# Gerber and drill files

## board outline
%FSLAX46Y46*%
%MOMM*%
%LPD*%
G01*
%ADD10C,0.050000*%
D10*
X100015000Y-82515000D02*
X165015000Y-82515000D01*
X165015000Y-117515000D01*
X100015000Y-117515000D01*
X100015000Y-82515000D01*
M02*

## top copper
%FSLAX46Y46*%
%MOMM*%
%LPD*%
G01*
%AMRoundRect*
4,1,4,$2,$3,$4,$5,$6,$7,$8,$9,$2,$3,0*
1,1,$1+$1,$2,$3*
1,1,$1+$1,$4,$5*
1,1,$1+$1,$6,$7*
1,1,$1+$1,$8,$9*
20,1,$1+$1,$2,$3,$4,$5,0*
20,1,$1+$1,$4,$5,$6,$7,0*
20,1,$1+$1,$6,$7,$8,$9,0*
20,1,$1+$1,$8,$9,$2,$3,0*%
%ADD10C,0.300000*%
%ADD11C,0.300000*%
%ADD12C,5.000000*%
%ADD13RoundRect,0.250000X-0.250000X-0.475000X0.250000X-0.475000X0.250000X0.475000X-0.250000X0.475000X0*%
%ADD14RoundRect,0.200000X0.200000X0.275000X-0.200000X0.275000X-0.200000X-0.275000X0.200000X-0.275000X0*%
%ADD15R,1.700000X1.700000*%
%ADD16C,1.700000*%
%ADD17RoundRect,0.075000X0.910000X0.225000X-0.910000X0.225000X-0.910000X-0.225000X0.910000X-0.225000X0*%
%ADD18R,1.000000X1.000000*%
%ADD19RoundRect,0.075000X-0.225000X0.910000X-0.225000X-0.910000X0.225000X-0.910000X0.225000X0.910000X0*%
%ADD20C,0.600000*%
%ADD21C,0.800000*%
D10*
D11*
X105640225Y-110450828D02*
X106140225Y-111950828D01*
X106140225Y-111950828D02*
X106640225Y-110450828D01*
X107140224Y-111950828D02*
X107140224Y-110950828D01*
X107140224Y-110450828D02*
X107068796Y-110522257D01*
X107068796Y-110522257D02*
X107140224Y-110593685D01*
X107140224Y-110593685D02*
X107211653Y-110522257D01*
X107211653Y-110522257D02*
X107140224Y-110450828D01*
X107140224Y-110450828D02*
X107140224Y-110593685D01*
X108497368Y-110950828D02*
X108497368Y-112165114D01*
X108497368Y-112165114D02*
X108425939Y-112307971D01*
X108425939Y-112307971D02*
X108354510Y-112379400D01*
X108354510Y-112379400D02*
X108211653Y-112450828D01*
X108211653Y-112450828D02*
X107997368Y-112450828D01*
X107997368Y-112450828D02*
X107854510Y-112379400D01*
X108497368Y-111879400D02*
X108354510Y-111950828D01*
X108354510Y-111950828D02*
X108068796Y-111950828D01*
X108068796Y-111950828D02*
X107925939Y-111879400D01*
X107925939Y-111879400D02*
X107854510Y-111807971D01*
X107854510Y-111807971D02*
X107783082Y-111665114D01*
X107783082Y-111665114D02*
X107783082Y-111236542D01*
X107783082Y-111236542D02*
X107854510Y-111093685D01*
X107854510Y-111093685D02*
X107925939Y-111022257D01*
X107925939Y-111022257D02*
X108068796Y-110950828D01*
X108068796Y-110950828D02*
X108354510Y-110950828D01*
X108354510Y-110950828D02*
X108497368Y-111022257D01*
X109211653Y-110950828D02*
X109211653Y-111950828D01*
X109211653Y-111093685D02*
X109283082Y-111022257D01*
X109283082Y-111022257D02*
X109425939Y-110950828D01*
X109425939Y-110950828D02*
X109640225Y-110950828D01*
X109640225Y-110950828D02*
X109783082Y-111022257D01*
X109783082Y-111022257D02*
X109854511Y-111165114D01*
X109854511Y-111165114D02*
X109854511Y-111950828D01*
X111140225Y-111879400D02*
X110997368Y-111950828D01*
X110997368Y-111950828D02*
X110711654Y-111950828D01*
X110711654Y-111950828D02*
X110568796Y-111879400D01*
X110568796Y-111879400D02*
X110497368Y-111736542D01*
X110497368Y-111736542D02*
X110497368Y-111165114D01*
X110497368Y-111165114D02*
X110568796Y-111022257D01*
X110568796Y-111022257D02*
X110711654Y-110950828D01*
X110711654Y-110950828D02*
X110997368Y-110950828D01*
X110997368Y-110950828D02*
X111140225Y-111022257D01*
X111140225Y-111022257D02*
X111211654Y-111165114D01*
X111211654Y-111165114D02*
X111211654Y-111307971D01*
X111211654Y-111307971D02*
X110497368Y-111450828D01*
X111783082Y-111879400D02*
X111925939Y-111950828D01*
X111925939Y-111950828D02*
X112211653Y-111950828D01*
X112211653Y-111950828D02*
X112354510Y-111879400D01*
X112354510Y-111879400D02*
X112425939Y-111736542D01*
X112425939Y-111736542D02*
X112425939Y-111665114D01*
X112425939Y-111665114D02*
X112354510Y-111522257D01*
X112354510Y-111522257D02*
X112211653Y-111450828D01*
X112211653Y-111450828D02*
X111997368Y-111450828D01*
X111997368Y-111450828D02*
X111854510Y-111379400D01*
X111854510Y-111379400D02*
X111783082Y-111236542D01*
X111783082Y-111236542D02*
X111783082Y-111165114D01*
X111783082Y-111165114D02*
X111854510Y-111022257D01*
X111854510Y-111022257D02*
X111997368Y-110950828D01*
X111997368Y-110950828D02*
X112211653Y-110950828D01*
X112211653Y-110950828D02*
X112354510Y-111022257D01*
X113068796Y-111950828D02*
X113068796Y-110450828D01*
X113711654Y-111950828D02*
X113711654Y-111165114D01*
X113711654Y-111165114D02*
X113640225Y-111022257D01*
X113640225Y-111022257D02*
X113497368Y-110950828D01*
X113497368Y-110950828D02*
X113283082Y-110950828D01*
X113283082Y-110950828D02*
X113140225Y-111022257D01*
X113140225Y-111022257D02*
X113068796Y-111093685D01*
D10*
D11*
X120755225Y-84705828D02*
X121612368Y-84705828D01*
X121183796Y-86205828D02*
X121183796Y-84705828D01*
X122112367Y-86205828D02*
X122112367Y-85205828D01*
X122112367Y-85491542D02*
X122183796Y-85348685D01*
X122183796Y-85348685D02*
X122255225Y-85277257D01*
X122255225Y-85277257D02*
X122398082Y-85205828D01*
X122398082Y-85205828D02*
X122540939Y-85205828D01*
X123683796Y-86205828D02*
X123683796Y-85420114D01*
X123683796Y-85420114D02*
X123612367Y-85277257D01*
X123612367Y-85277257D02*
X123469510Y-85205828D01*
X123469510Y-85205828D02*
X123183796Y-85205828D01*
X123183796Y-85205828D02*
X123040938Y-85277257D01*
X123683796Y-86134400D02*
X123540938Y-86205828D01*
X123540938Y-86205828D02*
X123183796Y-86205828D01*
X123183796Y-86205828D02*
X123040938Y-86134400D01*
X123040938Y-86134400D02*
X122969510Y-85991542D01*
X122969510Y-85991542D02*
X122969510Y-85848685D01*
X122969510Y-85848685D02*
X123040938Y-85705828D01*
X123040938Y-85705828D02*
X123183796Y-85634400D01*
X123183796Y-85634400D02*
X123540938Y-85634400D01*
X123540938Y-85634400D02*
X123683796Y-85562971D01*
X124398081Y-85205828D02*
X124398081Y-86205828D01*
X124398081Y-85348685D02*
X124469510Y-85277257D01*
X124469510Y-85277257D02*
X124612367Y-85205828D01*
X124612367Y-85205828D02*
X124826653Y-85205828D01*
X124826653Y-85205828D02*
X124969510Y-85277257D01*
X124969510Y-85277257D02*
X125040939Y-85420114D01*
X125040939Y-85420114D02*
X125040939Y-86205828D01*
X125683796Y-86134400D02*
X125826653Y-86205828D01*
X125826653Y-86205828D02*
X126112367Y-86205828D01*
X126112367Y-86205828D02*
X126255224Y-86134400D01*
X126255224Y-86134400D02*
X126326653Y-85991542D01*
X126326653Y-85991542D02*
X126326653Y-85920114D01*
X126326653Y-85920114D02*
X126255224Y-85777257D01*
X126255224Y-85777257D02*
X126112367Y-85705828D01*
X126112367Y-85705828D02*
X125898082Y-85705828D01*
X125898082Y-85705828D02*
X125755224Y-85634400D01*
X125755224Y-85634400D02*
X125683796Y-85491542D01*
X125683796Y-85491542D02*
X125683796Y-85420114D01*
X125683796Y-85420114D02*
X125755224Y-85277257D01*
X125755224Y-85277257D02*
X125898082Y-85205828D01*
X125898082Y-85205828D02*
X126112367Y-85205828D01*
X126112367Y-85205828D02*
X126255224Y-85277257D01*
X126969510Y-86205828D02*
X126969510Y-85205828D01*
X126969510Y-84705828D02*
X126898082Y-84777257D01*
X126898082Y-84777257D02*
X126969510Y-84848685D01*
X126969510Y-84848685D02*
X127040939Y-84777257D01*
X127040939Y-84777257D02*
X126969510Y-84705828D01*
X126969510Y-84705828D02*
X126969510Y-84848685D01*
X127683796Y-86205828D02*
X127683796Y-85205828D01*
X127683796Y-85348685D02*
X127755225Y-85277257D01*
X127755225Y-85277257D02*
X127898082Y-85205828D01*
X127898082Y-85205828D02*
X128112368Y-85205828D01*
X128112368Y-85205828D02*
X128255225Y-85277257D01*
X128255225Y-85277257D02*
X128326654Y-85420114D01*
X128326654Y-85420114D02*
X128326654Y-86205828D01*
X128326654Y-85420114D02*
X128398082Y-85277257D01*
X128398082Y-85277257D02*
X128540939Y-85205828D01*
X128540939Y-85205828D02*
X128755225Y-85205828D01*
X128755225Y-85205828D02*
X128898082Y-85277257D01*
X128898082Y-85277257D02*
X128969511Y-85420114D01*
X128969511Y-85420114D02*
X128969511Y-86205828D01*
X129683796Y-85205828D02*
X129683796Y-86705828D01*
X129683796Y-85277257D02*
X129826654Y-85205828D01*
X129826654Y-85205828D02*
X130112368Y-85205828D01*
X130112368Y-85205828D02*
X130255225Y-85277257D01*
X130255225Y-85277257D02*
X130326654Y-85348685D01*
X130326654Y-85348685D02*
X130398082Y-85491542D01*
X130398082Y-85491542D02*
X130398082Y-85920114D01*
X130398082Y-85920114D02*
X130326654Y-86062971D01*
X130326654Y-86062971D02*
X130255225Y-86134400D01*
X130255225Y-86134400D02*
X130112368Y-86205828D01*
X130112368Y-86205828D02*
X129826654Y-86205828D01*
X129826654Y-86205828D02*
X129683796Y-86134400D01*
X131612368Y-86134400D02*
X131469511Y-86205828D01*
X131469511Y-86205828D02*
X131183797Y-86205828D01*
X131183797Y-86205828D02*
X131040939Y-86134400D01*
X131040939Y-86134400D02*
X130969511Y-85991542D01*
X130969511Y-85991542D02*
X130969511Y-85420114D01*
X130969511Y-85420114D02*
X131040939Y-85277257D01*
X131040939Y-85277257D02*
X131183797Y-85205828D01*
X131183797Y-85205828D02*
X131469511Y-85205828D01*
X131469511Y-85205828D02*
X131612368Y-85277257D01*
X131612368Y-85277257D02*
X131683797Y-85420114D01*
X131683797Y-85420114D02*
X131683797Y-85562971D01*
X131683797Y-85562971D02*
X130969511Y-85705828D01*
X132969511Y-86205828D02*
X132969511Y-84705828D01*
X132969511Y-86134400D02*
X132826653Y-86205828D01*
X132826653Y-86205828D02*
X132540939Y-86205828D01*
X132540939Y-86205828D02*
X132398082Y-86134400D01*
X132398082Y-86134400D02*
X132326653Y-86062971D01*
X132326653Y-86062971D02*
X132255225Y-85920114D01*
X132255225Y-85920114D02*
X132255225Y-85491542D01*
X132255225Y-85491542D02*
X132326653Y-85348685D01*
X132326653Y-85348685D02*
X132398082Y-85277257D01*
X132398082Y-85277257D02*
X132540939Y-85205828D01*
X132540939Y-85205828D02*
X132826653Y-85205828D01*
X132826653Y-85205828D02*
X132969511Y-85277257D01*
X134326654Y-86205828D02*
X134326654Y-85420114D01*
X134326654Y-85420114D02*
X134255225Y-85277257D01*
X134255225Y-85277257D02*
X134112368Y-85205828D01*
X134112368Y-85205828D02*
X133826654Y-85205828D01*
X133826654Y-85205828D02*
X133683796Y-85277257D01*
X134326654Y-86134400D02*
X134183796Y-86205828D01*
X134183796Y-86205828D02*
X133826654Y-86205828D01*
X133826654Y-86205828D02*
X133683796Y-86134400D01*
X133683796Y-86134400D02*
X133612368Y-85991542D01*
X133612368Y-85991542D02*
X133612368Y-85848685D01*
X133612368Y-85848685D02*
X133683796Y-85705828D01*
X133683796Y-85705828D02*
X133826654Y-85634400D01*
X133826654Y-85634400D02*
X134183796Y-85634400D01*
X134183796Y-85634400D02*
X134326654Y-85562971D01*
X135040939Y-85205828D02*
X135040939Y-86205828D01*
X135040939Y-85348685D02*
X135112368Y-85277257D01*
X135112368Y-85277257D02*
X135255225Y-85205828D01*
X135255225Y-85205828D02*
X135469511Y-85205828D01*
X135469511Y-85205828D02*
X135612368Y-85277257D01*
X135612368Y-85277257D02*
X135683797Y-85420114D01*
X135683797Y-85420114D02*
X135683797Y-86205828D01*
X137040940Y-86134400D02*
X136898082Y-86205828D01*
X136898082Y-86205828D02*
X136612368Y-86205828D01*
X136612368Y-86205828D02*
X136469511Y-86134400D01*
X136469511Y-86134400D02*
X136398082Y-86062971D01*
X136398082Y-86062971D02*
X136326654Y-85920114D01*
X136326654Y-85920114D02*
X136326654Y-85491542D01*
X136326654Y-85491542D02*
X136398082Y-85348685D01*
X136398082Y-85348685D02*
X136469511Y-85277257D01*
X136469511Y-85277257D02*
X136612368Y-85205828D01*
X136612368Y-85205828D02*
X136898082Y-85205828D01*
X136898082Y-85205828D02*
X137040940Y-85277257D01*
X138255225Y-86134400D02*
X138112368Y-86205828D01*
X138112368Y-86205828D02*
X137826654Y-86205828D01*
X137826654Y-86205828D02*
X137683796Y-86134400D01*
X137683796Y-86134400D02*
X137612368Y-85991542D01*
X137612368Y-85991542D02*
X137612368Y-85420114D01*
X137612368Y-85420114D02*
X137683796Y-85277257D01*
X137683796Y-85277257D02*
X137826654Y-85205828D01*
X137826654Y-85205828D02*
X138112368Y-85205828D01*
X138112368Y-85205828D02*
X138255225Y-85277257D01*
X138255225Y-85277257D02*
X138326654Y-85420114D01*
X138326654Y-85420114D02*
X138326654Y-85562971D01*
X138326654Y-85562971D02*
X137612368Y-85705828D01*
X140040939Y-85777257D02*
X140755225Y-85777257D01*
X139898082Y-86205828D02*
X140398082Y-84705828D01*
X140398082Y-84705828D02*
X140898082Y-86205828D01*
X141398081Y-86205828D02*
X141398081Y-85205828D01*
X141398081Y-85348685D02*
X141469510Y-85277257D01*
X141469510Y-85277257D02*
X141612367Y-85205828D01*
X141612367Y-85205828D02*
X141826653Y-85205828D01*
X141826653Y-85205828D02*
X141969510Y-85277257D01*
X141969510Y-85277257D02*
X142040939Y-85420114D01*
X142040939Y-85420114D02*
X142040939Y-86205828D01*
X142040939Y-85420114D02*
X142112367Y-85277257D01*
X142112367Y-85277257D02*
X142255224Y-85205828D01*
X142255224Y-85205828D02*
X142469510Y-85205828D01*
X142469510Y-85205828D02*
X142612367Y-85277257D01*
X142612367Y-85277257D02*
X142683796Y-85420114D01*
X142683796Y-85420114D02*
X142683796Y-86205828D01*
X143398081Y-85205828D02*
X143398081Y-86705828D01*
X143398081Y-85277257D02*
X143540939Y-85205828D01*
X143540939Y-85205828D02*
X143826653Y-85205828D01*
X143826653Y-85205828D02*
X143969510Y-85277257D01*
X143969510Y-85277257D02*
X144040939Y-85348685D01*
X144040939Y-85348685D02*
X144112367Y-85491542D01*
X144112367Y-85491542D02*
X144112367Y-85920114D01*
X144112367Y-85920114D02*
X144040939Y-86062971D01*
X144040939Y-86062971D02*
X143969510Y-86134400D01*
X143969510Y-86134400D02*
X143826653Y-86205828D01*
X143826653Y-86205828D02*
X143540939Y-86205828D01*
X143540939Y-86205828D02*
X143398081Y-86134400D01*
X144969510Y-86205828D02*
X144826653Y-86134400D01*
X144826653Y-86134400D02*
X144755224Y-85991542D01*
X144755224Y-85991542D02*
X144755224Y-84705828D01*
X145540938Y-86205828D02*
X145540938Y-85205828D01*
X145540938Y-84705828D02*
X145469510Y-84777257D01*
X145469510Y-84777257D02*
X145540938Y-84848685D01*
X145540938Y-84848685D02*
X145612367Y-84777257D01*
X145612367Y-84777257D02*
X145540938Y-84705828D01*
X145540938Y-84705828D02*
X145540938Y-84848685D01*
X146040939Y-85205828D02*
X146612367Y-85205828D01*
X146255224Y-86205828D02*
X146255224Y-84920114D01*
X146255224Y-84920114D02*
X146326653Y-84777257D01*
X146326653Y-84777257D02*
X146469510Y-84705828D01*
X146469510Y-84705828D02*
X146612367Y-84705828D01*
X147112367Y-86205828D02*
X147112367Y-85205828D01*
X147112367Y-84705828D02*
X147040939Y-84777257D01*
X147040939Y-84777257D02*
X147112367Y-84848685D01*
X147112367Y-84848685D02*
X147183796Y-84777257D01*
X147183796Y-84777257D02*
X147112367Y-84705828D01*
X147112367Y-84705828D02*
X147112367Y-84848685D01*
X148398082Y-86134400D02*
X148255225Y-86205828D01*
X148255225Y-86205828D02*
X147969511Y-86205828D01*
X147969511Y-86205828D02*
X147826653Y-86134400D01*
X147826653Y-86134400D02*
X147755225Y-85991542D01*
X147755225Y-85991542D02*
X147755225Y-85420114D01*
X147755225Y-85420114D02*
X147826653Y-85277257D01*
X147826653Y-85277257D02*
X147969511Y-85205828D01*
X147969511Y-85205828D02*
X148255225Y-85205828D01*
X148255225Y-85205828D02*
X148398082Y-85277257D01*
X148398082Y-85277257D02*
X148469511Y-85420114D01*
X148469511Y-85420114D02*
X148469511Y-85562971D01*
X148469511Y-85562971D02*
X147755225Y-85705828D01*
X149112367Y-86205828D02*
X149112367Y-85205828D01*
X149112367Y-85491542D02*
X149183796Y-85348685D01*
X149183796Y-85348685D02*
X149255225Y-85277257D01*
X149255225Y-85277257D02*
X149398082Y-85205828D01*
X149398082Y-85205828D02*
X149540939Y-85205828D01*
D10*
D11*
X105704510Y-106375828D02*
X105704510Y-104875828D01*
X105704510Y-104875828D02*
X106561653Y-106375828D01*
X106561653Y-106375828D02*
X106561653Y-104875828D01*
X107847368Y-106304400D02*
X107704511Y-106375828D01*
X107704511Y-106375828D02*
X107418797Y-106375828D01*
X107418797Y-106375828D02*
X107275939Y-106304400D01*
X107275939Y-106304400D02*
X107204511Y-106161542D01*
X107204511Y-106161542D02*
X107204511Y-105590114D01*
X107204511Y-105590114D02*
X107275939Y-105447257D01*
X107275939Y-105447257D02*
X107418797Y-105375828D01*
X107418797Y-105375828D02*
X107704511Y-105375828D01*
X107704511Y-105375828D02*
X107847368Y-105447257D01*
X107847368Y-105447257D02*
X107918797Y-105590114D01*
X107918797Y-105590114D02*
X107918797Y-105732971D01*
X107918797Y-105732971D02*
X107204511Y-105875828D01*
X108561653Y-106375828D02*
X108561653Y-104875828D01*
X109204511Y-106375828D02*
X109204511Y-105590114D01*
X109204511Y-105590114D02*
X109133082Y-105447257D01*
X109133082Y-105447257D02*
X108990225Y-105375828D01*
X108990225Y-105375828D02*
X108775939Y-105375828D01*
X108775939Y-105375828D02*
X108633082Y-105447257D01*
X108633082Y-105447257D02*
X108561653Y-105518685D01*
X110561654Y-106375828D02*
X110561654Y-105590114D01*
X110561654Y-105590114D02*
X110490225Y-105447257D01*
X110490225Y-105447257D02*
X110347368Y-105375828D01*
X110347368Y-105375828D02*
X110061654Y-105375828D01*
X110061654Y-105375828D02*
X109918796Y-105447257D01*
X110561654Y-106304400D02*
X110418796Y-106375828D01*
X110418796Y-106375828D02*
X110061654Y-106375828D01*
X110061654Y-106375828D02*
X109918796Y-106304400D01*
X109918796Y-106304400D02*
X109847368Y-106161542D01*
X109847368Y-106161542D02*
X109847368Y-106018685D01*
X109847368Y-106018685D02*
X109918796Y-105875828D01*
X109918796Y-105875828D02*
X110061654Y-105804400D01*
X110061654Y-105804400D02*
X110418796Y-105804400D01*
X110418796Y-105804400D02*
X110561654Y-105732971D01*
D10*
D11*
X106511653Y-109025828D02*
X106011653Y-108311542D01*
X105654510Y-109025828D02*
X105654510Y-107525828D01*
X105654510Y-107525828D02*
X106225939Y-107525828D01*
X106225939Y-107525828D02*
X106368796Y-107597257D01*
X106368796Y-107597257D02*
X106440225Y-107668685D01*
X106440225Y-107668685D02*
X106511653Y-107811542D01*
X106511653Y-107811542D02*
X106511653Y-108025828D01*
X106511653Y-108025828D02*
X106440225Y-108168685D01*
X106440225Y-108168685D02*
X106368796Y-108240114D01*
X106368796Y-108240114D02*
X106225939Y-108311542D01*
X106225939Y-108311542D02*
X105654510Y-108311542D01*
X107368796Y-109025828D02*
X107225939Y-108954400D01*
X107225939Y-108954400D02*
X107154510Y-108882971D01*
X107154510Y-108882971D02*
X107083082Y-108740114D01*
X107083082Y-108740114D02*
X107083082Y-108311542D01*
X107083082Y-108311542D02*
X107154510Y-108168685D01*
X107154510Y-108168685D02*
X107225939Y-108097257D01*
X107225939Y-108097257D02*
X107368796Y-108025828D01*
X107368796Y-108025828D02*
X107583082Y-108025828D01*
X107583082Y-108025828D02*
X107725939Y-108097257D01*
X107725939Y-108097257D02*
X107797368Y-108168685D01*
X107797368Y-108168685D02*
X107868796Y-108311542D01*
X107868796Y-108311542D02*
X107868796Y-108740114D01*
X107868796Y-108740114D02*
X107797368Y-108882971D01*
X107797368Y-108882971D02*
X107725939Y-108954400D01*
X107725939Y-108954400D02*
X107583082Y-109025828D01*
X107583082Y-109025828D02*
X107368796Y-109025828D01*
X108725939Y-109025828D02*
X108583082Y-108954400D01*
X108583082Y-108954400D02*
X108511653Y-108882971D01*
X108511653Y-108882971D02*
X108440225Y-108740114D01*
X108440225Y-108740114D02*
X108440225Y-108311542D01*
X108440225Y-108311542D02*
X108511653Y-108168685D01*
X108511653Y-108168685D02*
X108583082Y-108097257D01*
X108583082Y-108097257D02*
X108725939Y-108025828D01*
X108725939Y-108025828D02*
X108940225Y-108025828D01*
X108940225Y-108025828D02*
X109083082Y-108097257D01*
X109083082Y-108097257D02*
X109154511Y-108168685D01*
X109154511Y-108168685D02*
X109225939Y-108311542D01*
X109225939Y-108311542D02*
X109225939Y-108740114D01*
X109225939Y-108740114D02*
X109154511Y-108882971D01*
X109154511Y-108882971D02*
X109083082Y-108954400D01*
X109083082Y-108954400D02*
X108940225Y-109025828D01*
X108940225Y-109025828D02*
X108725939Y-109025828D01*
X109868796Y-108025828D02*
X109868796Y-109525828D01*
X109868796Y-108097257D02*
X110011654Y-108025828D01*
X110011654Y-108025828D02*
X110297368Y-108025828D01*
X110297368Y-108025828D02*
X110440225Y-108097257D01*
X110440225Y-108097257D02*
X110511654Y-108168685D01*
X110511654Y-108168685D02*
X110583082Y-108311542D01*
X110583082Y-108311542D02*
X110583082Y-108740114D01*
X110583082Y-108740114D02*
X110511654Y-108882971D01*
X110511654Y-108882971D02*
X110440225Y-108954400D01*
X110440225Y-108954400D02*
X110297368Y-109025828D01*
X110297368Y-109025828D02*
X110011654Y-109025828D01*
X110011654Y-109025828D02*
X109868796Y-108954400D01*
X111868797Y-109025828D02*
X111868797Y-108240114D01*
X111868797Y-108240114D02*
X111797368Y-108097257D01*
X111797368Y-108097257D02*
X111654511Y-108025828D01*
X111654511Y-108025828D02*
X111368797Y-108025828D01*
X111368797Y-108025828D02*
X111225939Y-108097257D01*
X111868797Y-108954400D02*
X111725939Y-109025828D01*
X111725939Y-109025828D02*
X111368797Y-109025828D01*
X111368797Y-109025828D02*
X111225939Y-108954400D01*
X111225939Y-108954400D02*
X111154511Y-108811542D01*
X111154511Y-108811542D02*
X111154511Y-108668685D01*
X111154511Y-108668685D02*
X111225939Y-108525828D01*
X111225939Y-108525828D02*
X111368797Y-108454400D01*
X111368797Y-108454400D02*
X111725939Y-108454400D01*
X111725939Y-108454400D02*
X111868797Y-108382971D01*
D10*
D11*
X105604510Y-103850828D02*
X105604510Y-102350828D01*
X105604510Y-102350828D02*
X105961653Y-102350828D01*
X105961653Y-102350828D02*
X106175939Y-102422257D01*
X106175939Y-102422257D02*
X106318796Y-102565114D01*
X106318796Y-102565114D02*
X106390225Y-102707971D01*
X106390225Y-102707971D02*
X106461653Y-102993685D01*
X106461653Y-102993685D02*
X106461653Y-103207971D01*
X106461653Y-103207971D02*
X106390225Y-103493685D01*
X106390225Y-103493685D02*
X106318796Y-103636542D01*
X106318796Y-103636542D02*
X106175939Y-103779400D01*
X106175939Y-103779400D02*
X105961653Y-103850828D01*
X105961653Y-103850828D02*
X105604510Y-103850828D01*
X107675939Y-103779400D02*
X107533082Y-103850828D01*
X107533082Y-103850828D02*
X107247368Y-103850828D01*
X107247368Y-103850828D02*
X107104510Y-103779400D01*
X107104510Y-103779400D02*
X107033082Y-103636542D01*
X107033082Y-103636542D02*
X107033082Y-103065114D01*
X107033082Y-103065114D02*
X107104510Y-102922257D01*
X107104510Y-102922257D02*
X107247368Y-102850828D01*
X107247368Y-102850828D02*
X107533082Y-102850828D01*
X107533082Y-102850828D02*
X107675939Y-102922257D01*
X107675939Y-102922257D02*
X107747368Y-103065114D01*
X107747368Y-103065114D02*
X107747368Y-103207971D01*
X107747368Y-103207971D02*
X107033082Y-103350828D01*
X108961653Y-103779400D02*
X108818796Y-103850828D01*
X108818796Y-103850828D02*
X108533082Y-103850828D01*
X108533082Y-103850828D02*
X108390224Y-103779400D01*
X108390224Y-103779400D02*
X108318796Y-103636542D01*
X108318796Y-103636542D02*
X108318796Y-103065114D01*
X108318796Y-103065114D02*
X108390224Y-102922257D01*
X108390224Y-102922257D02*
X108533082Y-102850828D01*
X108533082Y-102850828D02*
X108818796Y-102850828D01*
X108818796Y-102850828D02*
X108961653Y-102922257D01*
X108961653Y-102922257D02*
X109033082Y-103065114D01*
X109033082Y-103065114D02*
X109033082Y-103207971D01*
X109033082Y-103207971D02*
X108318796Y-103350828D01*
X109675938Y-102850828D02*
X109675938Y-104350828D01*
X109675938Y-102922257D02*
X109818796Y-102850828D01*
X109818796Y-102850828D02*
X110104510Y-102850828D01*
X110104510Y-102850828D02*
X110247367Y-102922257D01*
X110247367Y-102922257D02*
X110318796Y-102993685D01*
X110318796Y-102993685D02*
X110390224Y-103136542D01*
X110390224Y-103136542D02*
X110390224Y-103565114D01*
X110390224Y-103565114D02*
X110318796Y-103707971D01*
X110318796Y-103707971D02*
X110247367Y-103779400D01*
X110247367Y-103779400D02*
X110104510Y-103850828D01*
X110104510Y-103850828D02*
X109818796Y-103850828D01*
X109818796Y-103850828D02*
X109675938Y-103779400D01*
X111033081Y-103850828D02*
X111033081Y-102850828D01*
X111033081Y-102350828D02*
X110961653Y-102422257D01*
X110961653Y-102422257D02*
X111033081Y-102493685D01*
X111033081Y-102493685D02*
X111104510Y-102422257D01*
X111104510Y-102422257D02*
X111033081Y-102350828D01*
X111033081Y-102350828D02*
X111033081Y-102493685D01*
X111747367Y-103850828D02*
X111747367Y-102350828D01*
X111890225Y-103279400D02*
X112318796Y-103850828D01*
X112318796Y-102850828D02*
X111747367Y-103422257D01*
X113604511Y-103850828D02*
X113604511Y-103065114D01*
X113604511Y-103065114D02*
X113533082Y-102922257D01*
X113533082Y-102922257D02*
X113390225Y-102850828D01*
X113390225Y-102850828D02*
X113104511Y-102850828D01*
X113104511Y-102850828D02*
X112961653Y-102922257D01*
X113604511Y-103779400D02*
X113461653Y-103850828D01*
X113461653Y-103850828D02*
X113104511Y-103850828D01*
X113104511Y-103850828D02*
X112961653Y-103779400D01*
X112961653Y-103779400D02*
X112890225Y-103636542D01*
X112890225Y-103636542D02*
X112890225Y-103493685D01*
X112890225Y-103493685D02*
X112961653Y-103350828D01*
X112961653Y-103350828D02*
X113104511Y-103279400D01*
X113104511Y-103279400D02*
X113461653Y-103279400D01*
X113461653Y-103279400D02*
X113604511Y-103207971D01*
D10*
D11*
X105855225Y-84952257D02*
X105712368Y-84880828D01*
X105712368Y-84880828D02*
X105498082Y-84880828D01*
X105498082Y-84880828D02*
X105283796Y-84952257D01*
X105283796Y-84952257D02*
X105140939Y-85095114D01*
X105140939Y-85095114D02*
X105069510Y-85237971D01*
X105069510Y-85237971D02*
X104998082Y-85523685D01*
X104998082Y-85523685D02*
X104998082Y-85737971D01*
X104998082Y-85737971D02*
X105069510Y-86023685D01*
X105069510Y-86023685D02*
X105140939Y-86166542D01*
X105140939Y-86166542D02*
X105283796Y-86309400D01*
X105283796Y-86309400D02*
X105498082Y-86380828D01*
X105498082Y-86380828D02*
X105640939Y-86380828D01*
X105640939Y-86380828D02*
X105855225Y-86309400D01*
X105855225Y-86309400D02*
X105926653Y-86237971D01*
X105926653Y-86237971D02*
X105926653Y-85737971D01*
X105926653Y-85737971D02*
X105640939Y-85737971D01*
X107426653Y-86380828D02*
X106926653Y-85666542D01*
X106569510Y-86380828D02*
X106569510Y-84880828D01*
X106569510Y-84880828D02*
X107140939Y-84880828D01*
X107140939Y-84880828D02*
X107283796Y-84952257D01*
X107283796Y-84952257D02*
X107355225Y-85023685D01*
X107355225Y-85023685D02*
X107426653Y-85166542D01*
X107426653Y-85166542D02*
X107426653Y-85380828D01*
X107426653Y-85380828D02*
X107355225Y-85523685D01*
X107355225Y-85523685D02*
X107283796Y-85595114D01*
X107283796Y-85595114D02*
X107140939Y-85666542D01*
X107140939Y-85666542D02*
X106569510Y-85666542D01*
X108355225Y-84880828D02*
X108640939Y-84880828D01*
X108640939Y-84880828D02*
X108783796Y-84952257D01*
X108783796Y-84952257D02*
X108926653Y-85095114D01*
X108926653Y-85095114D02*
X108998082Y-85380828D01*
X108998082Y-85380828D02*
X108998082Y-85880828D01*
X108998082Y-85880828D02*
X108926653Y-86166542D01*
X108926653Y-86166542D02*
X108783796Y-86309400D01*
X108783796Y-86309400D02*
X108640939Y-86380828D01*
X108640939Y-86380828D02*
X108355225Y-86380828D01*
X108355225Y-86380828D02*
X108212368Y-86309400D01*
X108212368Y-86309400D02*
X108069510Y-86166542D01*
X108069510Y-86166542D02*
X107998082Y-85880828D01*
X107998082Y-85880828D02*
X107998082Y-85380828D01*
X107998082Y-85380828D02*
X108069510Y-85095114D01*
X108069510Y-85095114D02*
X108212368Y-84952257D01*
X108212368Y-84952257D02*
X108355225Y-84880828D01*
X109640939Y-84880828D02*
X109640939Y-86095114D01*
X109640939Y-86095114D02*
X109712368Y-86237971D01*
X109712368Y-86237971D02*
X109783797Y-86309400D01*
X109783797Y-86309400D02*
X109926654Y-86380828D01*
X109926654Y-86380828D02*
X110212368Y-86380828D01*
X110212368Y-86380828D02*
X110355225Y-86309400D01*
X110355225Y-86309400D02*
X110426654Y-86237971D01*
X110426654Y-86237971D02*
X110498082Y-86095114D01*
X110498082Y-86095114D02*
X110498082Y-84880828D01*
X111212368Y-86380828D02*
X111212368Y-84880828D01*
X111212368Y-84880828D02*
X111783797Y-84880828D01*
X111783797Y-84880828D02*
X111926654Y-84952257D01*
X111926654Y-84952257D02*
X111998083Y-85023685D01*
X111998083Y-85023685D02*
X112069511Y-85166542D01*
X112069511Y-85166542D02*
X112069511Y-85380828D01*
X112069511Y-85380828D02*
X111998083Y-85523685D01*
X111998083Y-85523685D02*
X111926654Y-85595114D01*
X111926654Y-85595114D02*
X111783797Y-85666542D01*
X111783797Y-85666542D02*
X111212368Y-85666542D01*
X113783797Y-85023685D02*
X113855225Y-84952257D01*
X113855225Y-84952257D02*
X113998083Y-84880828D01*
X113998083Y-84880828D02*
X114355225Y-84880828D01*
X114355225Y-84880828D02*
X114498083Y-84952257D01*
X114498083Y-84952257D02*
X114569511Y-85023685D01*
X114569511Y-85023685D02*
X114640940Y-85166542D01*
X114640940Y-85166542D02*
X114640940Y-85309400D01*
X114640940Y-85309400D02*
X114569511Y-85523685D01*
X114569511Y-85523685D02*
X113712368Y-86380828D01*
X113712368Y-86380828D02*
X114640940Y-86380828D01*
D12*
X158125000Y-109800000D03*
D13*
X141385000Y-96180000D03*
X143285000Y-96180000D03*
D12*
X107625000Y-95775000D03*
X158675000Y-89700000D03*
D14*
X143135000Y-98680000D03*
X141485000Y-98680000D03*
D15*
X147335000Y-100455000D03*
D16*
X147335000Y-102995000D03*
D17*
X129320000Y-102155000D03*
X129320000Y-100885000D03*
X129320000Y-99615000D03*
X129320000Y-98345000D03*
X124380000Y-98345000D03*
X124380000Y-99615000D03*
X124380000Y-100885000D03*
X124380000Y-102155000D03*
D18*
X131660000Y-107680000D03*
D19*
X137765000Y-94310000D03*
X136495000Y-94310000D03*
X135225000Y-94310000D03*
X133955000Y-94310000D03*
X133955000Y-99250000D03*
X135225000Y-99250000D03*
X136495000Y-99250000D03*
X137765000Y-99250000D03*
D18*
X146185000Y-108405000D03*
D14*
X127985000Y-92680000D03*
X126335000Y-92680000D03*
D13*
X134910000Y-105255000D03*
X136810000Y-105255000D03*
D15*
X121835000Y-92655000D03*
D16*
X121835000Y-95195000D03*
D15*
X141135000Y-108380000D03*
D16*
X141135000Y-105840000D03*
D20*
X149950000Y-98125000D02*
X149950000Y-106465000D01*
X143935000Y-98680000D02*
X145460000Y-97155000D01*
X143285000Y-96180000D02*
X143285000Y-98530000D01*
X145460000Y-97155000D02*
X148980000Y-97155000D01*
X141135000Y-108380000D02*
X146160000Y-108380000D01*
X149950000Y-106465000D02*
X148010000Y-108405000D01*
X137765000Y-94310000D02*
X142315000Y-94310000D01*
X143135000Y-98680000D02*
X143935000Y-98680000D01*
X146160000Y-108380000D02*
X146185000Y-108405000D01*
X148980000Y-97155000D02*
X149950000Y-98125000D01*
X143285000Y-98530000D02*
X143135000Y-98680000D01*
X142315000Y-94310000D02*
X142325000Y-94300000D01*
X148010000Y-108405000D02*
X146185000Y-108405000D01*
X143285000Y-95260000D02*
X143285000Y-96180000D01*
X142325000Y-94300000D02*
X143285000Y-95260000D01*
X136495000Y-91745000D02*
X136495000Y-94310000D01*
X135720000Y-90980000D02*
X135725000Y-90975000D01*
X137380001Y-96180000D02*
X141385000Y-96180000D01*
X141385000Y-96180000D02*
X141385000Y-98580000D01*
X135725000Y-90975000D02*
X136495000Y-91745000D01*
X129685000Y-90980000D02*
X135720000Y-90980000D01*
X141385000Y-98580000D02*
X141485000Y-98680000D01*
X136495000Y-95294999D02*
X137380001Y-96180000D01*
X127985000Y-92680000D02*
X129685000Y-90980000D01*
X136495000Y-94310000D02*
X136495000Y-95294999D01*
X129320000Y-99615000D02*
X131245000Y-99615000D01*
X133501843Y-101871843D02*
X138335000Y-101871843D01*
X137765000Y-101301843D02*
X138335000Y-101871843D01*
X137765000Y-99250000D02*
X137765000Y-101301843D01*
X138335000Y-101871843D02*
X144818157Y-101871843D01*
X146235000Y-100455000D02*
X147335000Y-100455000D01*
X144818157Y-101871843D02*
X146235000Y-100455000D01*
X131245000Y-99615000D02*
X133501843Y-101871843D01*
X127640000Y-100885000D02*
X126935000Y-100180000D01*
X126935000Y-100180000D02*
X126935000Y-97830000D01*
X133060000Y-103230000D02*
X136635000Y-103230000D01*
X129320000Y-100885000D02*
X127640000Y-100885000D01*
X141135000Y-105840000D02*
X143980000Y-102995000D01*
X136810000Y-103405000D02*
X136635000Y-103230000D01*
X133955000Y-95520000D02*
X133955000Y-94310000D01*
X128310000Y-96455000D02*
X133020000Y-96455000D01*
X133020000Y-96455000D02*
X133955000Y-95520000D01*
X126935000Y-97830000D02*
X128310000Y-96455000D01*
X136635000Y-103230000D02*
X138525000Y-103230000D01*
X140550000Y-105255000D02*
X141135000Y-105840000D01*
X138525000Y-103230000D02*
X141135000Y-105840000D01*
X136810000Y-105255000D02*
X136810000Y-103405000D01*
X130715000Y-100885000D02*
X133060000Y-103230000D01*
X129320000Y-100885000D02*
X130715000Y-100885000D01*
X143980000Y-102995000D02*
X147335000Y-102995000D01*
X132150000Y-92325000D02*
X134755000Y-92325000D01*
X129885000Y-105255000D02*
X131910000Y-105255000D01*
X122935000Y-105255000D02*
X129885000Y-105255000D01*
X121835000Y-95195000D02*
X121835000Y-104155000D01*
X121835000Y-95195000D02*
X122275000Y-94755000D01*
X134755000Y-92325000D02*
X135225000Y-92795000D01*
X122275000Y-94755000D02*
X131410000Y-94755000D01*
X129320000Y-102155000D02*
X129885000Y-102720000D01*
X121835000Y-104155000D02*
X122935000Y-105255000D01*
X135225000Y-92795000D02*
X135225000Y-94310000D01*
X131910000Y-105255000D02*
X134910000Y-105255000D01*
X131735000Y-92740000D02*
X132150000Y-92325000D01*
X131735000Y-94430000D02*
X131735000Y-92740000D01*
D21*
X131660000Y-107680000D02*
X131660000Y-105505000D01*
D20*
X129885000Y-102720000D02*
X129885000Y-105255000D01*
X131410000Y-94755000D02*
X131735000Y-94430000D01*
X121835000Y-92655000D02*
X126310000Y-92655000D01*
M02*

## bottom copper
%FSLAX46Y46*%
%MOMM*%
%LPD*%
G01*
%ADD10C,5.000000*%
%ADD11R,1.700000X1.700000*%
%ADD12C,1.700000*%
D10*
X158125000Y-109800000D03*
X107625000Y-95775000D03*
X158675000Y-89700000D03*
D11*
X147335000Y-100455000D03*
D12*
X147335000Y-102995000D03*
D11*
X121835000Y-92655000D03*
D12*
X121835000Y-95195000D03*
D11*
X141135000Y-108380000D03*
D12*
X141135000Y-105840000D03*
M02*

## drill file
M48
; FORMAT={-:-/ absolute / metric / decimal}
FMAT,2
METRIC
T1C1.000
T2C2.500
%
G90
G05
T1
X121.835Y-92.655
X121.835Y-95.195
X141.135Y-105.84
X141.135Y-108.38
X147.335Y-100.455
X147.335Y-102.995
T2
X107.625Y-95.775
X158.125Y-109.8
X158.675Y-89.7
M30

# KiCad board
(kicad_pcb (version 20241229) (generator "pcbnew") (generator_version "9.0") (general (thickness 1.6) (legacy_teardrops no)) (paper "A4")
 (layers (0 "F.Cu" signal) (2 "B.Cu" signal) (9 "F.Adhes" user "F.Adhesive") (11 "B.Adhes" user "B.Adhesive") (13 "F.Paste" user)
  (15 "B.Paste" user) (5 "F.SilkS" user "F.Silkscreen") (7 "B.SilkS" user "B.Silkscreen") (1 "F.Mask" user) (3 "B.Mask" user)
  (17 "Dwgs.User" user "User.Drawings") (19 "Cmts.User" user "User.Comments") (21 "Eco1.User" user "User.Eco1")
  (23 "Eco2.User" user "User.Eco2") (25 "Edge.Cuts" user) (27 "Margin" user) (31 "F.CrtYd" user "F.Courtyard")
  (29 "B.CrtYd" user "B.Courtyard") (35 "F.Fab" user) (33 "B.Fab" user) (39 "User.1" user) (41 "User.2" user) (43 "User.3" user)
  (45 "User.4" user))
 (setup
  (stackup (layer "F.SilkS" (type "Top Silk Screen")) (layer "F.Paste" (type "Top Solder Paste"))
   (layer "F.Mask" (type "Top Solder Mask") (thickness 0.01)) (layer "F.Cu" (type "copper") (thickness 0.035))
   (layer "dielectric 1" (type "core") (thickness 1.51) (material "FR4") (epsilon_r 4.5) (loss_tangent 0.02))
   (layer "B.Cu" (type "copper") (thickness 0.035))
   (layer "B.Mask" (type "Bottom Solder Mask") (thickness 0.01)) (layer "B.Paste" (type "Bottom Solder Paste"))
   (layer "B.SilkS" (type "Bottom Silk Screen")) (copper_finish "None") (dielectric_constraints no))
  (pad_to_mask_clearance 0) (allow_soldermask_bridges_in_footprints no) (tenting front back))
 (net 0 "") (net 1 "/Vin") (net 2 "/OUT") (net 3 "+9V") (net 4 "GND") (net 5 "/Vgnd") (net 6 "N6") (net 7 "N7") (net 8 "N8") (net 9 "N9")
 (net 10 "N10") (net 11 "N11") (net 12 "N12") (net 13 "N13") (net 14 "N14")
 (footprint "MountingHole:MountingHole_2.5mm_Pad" (layer "F.Cu") (at 158.125 109.8)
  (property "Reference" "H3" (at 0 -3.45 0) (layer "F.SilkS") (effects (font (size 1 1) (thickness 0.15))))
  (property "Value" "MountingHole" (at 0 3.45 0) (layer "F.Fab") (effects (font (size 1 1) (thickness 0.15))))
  (pad "1" thru_hole circle (at 0 0) (size 5 5) (drill 2.5) (layers "*.Cu" "*.Mask") (remove_unused_layers no) (zone_connect 2)))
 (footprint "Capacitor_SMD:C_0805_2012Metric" (layer "F.Cu") (at 142.335 96.18)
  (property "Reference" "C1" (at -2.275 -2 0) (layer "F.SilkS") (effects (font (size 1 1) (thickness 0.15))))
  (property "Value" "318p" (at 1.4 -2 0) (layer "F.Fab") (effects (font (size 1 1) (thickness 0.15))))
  (pad "1" smd roundrect (at -0.95 0) (size 1 1.45) (layers "F.Cu" "F.Mask" "F.Paste") (roundrect_rratio 0.25) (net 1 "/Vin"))
  (pad "2" smd roundrect (at 0.95 0) (size 1 1.45) (layers "F.Cu" "F.Mask" "F.Paste") (roundrect_rratio 0.25) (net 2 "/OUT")))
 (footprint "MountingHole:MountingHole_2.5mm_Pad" (layer "F.Cu") (at 107.625 95.775)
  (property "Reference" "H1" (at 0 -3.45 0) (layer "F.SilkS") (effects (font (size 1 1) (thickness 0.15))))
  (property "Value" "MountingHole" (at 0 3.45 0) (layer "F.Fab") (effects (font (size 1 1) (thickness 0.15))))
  (pad "1" thru_hole circle (at 0 0) (size 5 5) (drill 2.5) (layers "*.Cu" "*.Mask") (remove_unused_layers no) (zone_connect 2)))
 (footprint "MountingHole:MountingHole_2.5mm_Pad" (layer "F.Cu") (at 158.675 89.7)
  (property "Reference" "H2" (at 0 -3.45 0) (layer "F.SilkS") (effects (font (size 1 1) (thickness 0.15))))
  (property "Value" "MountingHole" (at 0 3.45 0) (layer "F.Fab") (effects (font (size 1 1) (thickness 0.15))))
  (pad "1" thru_hole circle (at 0 0) (size 5 5) (drill 2.5) (layers "*.Cu" "*.Mask") (remove_unused_layers no) (zone_connect 2)))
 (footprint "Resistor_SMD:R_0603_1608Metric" (layer "F.Cu") (at 142.31 98.68 180)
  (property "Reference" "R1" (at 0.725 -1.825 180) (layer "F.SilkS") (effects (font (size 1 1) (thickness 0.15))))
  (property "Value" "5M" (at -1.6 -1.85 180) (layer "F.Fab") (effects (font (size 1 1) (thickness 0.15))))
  (pad "1" smd roundrect (at -0.825 0 180) (size 0.8 0.95) (layers "F.Cu" "F.Mask" "F.Paste") (roundrect_rratio 0.25) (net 2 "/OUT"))
  (pad "2" smd roundrect (at 0.825 0 180) (size 0.8 0.95) (layers "F.Cu" "F.Mask" "F.Paste") (roundrect_rratio 0.25) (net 1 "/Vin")))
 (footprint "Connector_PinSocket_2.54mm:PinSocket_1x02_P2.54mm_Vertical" (layer "F.Cu") (at 147.335 100.455)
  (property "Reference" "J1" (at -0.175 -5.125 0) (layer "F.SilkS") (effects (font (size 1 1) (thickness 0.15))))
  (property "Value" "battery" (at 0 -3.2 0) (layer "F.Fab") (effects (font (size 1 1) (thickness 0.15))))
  (pad "1" thru_hole rect (at 0 0) (size 1.7 1.7) (drill 1) (layers "*.Cu" "*.Mask") (remove_unused_layers no) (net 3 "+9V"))
  (pad "2" thru_hole circle (at 0 2.54) (size 1.7 1.7) (drill 1) (layers "*.Cu" "*.Mask") (remove_unused_layers no) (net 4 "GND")))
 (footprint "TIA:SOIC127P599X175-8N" (layer "F.Cu") (at 126.85 100.25 180)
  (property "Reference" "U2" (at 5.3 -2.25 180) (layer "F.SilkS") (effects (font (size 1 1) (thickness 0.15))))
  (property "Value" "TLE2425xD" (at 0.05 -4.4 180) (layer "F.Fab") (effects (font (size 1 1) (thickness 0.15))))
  (pad "1" smd roundrect (at -2.47 -1.905 180) (size 1.97 0.6) (layers "F.Cu" "F.Mask" "F.Paste") (roundrect_rratio 0.125) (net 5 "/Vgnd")
   (solder_mask_margin 0.102))
  (pad "2" smd roundrect (at -2.47 -0.635 180) (size 1.97 0.6) (layers "F.Cu" "F.Mask" "F.Paste") (roundrect_rratio 0.125) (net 4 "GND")
   (solder_mask_margin 0.102))
  (pad "3" smd roundrect (at -2.47 0.635 180) (size 1.97 0.6) (layers "F.Cu" "F.Mask" "F.Paste") (roundrect_rratio 0.125) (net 3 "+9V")
   (solder_mask_margin 0.102))
  (pad "4" smd roundrect (at -2.47 1.905 180) (size 1.97 0.6) (layers "F.Cu" "F.Mask" "F.Paste") (roundrect_rratio 0.125) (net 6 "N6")
   (solder_mask_margin 0.102))
  (pad "5" smd roundrect (at 2.47 1.905 180) (size 1.97 0.6) (layers "F.Cu" "F.Mask" "F.Paste") (roundrect_rratio 0.125) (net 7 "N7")
   (solder_mask_margin 0.102))
  (pad "6" smd roundrect (at 2.47 0.635 180) (size 1.97 0.6) (layers "F.Cu" "F.Mask" "F.Paste") (roundrect_rratio 0.125) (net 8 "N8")
   (solder_mask_margin 0.102))
  (pad "7" smd roundrect (at 2.47 -0.635 180) (size 1.97 0.6) (layers "F.Cu" "F.Mask" "F.Paste") (roundrect_rratio 0.125) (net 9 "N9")
   (solder_mask_margin 0.102))
  (pad "8" smd roundrect (at 2.47 -1.905 180) (size 1.97 0.6) (layers "F.Cu" "F.Mask" "F.Paste") (roundrect_rratio 0.125) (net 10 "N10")
   (solder_mask_margin 0.102)))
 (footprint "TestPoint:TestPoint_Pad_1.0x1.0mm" (layer "F.Cu") (at 131.66 107.68 180)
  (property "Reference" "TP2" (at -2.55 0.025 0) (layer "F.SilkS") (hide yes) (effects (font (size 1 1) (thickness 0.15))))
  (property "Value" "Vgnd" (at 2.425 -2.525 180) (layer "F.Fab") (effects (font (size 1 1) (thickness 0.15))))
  (pad "1" smd rect (at 0 0 180) (size 1 1) (layers "F.Cu" "F.Mask") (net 5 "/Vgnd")))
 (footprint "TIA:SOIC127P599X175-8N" (layer "F.Cu") (at 135.86 96.78 -90)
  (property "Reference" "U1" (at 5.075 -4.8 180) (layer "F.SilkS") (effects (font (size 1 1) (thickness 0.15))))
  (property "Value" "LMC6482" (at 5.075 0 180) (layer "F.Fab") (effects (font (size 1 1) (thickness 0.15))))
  (pad "1" smd roundrect (at -2.47 -1.905 270) (size 1.97 0.6) (layers "F.Cu" "F.Mask" "F.Paste") (roundrect_rratio 0.125) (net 2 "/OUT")
   (solder_mask_margin 0.102))
  (pad "2" smd roundrect (at -2.47 -0.635 270) (size 1.97 0.6) (layers "F.Cu" "F.Mask" "F.Paste") (roundrect_rratio 0.125) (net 1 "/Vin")
   (solder_mask_margin 0.102))
  (pad "3" smd roundrect (at -2.47 0.635 270) (size 1.97 0.6) (layers "F.Cu" "F.Mask" "F.Paste") (roundrect_rratio 0.125) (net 5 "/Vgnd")
   (solder_mask_margin 0.102))
  (pad "4" smd roundrect (at -2.47 1.905 270) (size 1.97 0.6) (layers "F.Cu" "F.Mask" "F.Paste") (roundrect_rratio 0.125) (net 4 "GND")
   (solder_mask_margin 0.102))
  (pad "5" smd roundrect (at 2.47 1.905 270) (size 1.97 0.6) (layers "F.Cu" "F.Mask" "F.Paste") (roundrect_rratio 0.125) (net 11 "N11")
   (solder_mask_margin 0.102))
  (pad "6" smd roundrect (at 2.47 0.635 270) (size 1.97 0.6) (layers "F.Cu" "F.Mask" "F.Paste") (roundrect_rratio 0.125) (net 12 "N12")
   (solder_mask_margin 0.102))
  (pad "7" smd roundrect (at 2.47 -0.635 270) (size 1.97 0.6) (layers "F.Cu" "F.Mask" "F.Paste") (roundrect_rratio 0.125) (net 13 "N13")
   (solder_mask_margin 0.102))
  (pad "8" smd roundrect (at 2.47 -1.905 270) (size 1.97 0.6) (layers "F.Cu" "F.Mask" "F.Paste") (roundrect_rratio 0.125) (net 3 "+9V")
   (solder_mask_margin 0.102)))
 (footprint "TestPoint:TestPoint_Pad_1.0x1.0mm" (layer "F.Cu") (at 146.185 108.405)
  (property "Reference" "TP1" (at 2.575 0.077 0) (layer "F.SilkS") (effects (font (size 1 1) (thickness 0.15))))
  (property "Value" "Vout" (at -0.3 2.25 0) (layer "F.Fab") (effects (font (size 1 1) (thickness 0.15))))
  (pad "1" smd rect (at 0 0) (size 1 1) (layers "F.Cu" "F.Mask") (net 2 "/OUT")))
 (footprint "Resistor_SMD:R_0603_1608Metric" (layer "F.Cu") (at 127.16 92.68 180)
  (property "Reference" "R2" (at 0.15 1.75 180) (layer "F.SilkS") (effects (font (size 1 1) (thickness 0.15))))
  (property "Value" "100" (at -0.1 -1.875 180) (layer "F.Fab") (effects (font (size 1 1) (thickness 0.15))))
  (pad "1" smd roundrect (at -0.825 0 180) (size 0.8 0.95) (layers "F.Cu" "F.Mask" "F.Paste") (roundrect_rratio 0.25) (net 1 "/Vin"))
  (pad "2" smd roundrect (at 0.825 0 180) (size 0.8 0.95) (layers "F.Cu" "F.Mask" "F.Paste") (roundrect_rratio 0.25) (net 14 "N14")))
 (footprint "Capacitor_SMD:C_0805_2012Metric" (layer "F.Cu") (at 135.86 105.255)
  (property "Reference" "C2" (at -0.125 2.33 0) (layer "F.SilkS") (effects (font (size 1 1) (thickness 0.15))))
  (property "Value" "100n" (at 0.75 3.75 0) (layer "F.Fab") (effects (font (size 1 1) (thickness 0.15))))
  (pad "1" smd roundrect (at -0.95 0) (size 1 1.45) (layers "F.Cu" "F.Mask" "F.Paste") (roundrect_rratio 0.25) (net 5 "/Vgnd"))
  (pad "2" smd roundrect (at 0.95 0) (size 1 1.45) (layers "F.Cu" "F.Mask" "F.Paste") (roundrect_rratio 0.25) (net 4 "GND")))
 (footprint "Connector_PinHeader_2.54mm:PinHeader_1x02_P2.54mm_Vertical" (layer "F.Cu") (at 121.835 92.655)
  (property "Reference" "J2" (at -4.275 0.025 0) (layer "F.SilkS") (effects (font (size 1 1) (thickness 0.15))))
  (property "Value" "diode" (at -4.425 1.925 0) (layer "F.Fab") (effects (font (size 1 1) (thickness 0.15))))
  (pad "1" thru_hole rect (at 0 0) (size 1.7 1.7) (drill 1) (layers "*.Cu" "*.Mask") (remove_unused_layers no) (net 14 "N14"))
  (pad "2" thru_hole circle (at 0 2.54) (size 1.7 1.7) (drill 1) (layers "*.Cu" "*.Mask") (remove_unused_layers no) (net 5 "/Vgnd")))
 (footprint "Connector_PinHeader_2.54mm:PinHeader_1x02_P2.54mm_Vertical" (layer "F.Cu") (at 141.135 108.38 180)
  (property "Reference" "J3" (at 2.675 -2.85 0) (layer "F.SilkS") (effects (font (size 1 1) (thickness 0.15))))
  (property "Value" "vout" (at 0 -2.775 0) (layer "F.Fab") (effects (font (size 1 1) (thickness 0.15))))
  (pad "1" thru_hole rect (at 0 0 180) (size 1.7 1.7) (drill 1) (layers "*.Cu" "*.Mask") (remove_unused_layers no) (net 2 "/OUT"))
  (pad "2" thru_hole circle (at 0 2.54 180) (size 1.7 1.7) (drill 1) (layers "*.Cu" "*.Mask") (remove_unused_layers no) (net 4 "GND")))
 (gr_rect (start 100.015 82.515) (end 165.015 117.515) (stroke (width 0.05) (type solid)) (fill no) (layer "Edge.Cuts"))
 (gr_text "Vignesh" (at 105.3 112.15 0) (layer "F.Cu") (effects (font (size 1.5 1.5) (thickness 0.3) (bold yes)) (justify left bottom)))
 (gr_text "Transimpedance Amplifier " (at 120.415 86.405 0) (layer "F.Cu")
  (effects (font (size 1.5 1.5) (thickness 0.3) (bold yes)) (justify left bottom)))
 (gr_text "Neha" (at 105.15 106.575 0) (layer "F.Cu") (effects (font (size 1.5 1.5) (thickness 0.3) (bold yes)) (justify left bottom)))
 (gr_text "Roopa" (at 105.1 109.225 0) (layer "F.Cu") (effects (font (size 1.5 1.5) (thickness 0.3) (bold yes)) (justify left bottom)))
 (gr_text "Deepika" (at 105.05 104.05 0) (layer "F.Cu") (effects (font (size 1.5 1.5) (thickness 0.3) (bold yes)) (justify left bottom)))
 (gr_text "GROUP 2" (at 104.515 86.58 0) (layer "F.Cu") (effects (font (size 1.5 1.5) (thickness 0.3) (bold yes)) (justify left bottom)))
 (segment (start 149.95 98.125) (end 149.95 106.465) (width 0.6) (layer "F.Cu") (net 2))
 (segment (start 143.935 98.68) (end 145.46 97.155) (width 0.6) (layer "F.Cu") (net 2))
 (segment (start 143.285 96.18) (end 143.285 98.53) (width 0.6) (layer "F.Cu") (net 2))
 (segment (start 145.46 97.155) (end 148.98 97.155) (width 0.6) (layer "F.Cu") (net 2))
 (segment (start 141.135 108.38) (end 146.16 108.38) (width 0.6) (layer "F.Cu") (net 2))
 (segment (start 149.95 106.465) (end 148.01 108.405) (width 0.6) (layer "F.Cu") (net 2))
 (segment (start 137.765 94.31) (end 142.315 94.31) (width 0.6) (layer "F.Cu") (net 2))
 (segment (start 143.135 98.68) (end 143.935 98.68) (width 0.6) (layer "F.Cu") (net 2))
 (segment (start 146.16 108.38) (end 146.185 108.405) (width 0.6) (layer "F.Cu") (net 2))
 (segment (start 148.98 97.155) (end 149.95 98.125) (width 0.6) (layer "F.Cu") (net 2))
 (segment (start 143.285 98.53) (end 143.135 98.68) (width 0.6) (layer "F.Cu") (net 2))
 (segment (start 142.315 94.31) (end 142.325 94.3) (width 0.6) (layer "F.Cu") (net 2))
 (segment (start 148.01 108.405) (end 146.185 108.405) (width 0.6) (layer "F.Cu") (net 2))
 (segment (start 143.285 95.26) (end 143.285 96.18) (width 0.6) (layer "F.Cu") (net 2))
 (segment (start 142.325 94.3) (end 143.285 95.26) (width 0.6) (layer "F.Cu") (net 2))
 (segment (start 136.495 91.745) (end 136.495 94.31) (width 0.6) (layer "F.Cu") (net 1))
 (segment (start 135.72 90.98) (end 135.725 90.975) (width 0.6) (layer "F.Cu") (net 1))
 (segment (start 137.380001 96.18) (end 141.385 96.18) (width 0.6) (layer "F.Cu") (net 1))
 (segment (start 141.385 96.18) (end 141.385 98.58) (width 0.6) (layer "F.Cu") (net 1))
 (segment (start 135.725 90.975) (end 136.495 91.745) (width 0.6) (layer "F.Cu") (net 1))
 (segment (start 129.685 90.98) (end 135.72 90.98) (width 0.6) (layer "F.Cu") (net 1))
 (segment (start 141.385 98.58) (end 141.485 98.68) (width 0.6) (layer "F.Cu") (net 1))
 (segment (start 136.495 95.294999) (end 137.380001 96.18) (width 0.6) (layer "F.Cu") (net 1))
 (segment (start 127.985 92.68) (end 129.685 90.98) (width 0.6) (layer "F.Cu") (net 1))
 (segment (start 136.495 94.31) (end 136.495 95.294999) (width 0.6) (layer "F.Cu") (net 1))
 (segment (start 129.32 99.615) (end 131.245 99.615) (width 0.6) (layer "F.Cu") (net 3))
 (segment (start 133.501843 101.871843) (end 138.335 101.871843) (width 0.6) (layer "F.Cu") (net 3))
 (segment (start 137.765 101.301843) (end 138.335 101.871843) (width 0.6) (layer "F.Cu") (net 3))
 (segment (start 137.765 99.25) (end 137.765 101.301843) (width 0.6) (layer "F.Cu") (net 3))
 (segment (start 138.335 101.871843) (end 144.818157 101.871843) (width 0.6) (layer "F.Cu") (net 3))
 (segment (start 146.235 100.455) (end 147.335 100.455) (width 0.6) (layer "F.Cu") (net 3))
 (segment (start 144.818157 101.871843) (end 146.235 100.455) (width 0.6) (layer "F.Cu") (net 3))
 (segment (start 131.245 99.615) (end 133.501843 101.871843) (width 0.6) (layer "F.Cu") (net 3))
 (segment (start 127.64 100.885) (end 126.935 100.18) (width 0.6) (layer "F.Cu") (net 4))
 (segment (start 126.935 100.18) (end 126.935 97.83) (width 0.6) (layer "F.Cu") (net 4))
 (segment (start 133.06 103.23) (end 136.635 103.23) (width 0.6) (layer "F.Cu") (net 4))
 (segment (start 129.32 100.885) (end 127.64 100.885) (width 0.6) (layer "F.Cu") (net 4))
 (segment (start 141.135 105.84) (end 143.98 102.995) (width 0.6) (layer "F.Cu") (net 4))
 (segment (start 136.81 103.405) (end 136.635 103.23) (width 0.6) (layer "F.Cu") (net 4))
 (segment (start 133.955 95.52) (end 133.955 94.31) (width 0.6) (layer "F.Cu") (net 4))
 (segment (start 128.31 96.455) (end 133.02 96.455) (width 0.6) (layer "F.Cu") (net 4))
 (segment (start 133.02 96.455) (end 133.955 95.52) (width 0.6) (layer "F.Cu") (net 4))
 (segment (start 126.935 97.83) (end 128.31 96.455) (width 0.6) (layer "F.Cu") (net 4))
 (segment (start 136.635 103.23) (end 138.525 103.23) (width 0.6) (layer "F.Cu") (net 4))
 (segment (start 140.55 105.255) (end 141.135 105.84) (width 0.6) (layer "F.Cu") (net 4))
 (segment (start 138.525 103.23) (end 141.135 105.84) (width 0.6) (layer "F.Cu") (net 4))
 (segment (start 136.81 105.255) (end 136.81 103.405) (width 0.6) (layer "F.Cu") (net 4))
 (segment (start 130.715 100.885) (end 133.06 103.23) (width 0.6) (layer "F.Cu") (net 4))
 (segment (start 129.32 100.885) (end 130.715 100.885) (width 0.6) (layer "F.Cu") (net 4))
 (segment (start 143.98 102.995) (end 147.335 102.995) (width 0.6) (layer "F.Cu") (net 4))
 (segment (start 132.15 92.325) (end 134.755 92.325) (width 0.6) (layer "F.Cu") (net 5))
 (segment (start 129.885 105.255) (end 131.91 105.255) (width 0.6) (layer "F.Cu") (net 5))
 (segment (start 122.935 105.255) (end 129.885 105.255) (width 0.6) (layer "F.Cu") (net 5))
 (segment (start 121.835 95.195) (end 121.835 104.155) (width 0.6) (layer "F.Cu") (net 5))
 (segment (start 121.835 95.195) (end 122.275 94.755) (width 0.6) (layer "F.Cu") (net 5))
 (segment (start 134.755 92.325) (end 135.225 92.795) (width 0.6) (layer "F.Cu") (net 5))
 (segment (start 122.275 94.755) (end 131.41 94.755) (width 0.6) (layer "F.Cu") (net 5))
 (segment (start 129.32 102.155) (end 129.885 102.72) (width 0.6) (layer "F.Cu") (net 5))
 (segment (start 121.835 104.155) (end 122.935 105.255) (width 0.6) (layer "F.Cu") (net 5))
 (segment (start 135.225 92.795) (end 135.225 94.31) (width 0.6) (layer "F.Cu") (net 5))
 (segment (start 131.91 105.255) (end 134.91 105.255) (width 0.6) (layer "F.Cu") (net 5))
 (segment (start 131.735 92.74) (end 132.15 92.325) (width 0.6) (layer "F.Cu") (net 5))
 (segment (start 131.735 94.43) (end 131.735 92.74) (width 0.6) (layer "F.Cu") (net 5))
 (segment (start 131.66 107.68) (end 131.66 105.505) (width 0.8) (layer "F.Cu") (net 5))
 (segment (start 129.885 102.72) (end 129.885 105.255) (width 0.6) (layer "F.Cu") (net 5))
 (segment (start 131.41 94.755) (end 131.735 94.43) (width 0.6) (layer "F.Cu") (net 5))
 (segment (start 121.835 92.655) (end 126.31 92.655) (width 0.6) (layer "F.Cu") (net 14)))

